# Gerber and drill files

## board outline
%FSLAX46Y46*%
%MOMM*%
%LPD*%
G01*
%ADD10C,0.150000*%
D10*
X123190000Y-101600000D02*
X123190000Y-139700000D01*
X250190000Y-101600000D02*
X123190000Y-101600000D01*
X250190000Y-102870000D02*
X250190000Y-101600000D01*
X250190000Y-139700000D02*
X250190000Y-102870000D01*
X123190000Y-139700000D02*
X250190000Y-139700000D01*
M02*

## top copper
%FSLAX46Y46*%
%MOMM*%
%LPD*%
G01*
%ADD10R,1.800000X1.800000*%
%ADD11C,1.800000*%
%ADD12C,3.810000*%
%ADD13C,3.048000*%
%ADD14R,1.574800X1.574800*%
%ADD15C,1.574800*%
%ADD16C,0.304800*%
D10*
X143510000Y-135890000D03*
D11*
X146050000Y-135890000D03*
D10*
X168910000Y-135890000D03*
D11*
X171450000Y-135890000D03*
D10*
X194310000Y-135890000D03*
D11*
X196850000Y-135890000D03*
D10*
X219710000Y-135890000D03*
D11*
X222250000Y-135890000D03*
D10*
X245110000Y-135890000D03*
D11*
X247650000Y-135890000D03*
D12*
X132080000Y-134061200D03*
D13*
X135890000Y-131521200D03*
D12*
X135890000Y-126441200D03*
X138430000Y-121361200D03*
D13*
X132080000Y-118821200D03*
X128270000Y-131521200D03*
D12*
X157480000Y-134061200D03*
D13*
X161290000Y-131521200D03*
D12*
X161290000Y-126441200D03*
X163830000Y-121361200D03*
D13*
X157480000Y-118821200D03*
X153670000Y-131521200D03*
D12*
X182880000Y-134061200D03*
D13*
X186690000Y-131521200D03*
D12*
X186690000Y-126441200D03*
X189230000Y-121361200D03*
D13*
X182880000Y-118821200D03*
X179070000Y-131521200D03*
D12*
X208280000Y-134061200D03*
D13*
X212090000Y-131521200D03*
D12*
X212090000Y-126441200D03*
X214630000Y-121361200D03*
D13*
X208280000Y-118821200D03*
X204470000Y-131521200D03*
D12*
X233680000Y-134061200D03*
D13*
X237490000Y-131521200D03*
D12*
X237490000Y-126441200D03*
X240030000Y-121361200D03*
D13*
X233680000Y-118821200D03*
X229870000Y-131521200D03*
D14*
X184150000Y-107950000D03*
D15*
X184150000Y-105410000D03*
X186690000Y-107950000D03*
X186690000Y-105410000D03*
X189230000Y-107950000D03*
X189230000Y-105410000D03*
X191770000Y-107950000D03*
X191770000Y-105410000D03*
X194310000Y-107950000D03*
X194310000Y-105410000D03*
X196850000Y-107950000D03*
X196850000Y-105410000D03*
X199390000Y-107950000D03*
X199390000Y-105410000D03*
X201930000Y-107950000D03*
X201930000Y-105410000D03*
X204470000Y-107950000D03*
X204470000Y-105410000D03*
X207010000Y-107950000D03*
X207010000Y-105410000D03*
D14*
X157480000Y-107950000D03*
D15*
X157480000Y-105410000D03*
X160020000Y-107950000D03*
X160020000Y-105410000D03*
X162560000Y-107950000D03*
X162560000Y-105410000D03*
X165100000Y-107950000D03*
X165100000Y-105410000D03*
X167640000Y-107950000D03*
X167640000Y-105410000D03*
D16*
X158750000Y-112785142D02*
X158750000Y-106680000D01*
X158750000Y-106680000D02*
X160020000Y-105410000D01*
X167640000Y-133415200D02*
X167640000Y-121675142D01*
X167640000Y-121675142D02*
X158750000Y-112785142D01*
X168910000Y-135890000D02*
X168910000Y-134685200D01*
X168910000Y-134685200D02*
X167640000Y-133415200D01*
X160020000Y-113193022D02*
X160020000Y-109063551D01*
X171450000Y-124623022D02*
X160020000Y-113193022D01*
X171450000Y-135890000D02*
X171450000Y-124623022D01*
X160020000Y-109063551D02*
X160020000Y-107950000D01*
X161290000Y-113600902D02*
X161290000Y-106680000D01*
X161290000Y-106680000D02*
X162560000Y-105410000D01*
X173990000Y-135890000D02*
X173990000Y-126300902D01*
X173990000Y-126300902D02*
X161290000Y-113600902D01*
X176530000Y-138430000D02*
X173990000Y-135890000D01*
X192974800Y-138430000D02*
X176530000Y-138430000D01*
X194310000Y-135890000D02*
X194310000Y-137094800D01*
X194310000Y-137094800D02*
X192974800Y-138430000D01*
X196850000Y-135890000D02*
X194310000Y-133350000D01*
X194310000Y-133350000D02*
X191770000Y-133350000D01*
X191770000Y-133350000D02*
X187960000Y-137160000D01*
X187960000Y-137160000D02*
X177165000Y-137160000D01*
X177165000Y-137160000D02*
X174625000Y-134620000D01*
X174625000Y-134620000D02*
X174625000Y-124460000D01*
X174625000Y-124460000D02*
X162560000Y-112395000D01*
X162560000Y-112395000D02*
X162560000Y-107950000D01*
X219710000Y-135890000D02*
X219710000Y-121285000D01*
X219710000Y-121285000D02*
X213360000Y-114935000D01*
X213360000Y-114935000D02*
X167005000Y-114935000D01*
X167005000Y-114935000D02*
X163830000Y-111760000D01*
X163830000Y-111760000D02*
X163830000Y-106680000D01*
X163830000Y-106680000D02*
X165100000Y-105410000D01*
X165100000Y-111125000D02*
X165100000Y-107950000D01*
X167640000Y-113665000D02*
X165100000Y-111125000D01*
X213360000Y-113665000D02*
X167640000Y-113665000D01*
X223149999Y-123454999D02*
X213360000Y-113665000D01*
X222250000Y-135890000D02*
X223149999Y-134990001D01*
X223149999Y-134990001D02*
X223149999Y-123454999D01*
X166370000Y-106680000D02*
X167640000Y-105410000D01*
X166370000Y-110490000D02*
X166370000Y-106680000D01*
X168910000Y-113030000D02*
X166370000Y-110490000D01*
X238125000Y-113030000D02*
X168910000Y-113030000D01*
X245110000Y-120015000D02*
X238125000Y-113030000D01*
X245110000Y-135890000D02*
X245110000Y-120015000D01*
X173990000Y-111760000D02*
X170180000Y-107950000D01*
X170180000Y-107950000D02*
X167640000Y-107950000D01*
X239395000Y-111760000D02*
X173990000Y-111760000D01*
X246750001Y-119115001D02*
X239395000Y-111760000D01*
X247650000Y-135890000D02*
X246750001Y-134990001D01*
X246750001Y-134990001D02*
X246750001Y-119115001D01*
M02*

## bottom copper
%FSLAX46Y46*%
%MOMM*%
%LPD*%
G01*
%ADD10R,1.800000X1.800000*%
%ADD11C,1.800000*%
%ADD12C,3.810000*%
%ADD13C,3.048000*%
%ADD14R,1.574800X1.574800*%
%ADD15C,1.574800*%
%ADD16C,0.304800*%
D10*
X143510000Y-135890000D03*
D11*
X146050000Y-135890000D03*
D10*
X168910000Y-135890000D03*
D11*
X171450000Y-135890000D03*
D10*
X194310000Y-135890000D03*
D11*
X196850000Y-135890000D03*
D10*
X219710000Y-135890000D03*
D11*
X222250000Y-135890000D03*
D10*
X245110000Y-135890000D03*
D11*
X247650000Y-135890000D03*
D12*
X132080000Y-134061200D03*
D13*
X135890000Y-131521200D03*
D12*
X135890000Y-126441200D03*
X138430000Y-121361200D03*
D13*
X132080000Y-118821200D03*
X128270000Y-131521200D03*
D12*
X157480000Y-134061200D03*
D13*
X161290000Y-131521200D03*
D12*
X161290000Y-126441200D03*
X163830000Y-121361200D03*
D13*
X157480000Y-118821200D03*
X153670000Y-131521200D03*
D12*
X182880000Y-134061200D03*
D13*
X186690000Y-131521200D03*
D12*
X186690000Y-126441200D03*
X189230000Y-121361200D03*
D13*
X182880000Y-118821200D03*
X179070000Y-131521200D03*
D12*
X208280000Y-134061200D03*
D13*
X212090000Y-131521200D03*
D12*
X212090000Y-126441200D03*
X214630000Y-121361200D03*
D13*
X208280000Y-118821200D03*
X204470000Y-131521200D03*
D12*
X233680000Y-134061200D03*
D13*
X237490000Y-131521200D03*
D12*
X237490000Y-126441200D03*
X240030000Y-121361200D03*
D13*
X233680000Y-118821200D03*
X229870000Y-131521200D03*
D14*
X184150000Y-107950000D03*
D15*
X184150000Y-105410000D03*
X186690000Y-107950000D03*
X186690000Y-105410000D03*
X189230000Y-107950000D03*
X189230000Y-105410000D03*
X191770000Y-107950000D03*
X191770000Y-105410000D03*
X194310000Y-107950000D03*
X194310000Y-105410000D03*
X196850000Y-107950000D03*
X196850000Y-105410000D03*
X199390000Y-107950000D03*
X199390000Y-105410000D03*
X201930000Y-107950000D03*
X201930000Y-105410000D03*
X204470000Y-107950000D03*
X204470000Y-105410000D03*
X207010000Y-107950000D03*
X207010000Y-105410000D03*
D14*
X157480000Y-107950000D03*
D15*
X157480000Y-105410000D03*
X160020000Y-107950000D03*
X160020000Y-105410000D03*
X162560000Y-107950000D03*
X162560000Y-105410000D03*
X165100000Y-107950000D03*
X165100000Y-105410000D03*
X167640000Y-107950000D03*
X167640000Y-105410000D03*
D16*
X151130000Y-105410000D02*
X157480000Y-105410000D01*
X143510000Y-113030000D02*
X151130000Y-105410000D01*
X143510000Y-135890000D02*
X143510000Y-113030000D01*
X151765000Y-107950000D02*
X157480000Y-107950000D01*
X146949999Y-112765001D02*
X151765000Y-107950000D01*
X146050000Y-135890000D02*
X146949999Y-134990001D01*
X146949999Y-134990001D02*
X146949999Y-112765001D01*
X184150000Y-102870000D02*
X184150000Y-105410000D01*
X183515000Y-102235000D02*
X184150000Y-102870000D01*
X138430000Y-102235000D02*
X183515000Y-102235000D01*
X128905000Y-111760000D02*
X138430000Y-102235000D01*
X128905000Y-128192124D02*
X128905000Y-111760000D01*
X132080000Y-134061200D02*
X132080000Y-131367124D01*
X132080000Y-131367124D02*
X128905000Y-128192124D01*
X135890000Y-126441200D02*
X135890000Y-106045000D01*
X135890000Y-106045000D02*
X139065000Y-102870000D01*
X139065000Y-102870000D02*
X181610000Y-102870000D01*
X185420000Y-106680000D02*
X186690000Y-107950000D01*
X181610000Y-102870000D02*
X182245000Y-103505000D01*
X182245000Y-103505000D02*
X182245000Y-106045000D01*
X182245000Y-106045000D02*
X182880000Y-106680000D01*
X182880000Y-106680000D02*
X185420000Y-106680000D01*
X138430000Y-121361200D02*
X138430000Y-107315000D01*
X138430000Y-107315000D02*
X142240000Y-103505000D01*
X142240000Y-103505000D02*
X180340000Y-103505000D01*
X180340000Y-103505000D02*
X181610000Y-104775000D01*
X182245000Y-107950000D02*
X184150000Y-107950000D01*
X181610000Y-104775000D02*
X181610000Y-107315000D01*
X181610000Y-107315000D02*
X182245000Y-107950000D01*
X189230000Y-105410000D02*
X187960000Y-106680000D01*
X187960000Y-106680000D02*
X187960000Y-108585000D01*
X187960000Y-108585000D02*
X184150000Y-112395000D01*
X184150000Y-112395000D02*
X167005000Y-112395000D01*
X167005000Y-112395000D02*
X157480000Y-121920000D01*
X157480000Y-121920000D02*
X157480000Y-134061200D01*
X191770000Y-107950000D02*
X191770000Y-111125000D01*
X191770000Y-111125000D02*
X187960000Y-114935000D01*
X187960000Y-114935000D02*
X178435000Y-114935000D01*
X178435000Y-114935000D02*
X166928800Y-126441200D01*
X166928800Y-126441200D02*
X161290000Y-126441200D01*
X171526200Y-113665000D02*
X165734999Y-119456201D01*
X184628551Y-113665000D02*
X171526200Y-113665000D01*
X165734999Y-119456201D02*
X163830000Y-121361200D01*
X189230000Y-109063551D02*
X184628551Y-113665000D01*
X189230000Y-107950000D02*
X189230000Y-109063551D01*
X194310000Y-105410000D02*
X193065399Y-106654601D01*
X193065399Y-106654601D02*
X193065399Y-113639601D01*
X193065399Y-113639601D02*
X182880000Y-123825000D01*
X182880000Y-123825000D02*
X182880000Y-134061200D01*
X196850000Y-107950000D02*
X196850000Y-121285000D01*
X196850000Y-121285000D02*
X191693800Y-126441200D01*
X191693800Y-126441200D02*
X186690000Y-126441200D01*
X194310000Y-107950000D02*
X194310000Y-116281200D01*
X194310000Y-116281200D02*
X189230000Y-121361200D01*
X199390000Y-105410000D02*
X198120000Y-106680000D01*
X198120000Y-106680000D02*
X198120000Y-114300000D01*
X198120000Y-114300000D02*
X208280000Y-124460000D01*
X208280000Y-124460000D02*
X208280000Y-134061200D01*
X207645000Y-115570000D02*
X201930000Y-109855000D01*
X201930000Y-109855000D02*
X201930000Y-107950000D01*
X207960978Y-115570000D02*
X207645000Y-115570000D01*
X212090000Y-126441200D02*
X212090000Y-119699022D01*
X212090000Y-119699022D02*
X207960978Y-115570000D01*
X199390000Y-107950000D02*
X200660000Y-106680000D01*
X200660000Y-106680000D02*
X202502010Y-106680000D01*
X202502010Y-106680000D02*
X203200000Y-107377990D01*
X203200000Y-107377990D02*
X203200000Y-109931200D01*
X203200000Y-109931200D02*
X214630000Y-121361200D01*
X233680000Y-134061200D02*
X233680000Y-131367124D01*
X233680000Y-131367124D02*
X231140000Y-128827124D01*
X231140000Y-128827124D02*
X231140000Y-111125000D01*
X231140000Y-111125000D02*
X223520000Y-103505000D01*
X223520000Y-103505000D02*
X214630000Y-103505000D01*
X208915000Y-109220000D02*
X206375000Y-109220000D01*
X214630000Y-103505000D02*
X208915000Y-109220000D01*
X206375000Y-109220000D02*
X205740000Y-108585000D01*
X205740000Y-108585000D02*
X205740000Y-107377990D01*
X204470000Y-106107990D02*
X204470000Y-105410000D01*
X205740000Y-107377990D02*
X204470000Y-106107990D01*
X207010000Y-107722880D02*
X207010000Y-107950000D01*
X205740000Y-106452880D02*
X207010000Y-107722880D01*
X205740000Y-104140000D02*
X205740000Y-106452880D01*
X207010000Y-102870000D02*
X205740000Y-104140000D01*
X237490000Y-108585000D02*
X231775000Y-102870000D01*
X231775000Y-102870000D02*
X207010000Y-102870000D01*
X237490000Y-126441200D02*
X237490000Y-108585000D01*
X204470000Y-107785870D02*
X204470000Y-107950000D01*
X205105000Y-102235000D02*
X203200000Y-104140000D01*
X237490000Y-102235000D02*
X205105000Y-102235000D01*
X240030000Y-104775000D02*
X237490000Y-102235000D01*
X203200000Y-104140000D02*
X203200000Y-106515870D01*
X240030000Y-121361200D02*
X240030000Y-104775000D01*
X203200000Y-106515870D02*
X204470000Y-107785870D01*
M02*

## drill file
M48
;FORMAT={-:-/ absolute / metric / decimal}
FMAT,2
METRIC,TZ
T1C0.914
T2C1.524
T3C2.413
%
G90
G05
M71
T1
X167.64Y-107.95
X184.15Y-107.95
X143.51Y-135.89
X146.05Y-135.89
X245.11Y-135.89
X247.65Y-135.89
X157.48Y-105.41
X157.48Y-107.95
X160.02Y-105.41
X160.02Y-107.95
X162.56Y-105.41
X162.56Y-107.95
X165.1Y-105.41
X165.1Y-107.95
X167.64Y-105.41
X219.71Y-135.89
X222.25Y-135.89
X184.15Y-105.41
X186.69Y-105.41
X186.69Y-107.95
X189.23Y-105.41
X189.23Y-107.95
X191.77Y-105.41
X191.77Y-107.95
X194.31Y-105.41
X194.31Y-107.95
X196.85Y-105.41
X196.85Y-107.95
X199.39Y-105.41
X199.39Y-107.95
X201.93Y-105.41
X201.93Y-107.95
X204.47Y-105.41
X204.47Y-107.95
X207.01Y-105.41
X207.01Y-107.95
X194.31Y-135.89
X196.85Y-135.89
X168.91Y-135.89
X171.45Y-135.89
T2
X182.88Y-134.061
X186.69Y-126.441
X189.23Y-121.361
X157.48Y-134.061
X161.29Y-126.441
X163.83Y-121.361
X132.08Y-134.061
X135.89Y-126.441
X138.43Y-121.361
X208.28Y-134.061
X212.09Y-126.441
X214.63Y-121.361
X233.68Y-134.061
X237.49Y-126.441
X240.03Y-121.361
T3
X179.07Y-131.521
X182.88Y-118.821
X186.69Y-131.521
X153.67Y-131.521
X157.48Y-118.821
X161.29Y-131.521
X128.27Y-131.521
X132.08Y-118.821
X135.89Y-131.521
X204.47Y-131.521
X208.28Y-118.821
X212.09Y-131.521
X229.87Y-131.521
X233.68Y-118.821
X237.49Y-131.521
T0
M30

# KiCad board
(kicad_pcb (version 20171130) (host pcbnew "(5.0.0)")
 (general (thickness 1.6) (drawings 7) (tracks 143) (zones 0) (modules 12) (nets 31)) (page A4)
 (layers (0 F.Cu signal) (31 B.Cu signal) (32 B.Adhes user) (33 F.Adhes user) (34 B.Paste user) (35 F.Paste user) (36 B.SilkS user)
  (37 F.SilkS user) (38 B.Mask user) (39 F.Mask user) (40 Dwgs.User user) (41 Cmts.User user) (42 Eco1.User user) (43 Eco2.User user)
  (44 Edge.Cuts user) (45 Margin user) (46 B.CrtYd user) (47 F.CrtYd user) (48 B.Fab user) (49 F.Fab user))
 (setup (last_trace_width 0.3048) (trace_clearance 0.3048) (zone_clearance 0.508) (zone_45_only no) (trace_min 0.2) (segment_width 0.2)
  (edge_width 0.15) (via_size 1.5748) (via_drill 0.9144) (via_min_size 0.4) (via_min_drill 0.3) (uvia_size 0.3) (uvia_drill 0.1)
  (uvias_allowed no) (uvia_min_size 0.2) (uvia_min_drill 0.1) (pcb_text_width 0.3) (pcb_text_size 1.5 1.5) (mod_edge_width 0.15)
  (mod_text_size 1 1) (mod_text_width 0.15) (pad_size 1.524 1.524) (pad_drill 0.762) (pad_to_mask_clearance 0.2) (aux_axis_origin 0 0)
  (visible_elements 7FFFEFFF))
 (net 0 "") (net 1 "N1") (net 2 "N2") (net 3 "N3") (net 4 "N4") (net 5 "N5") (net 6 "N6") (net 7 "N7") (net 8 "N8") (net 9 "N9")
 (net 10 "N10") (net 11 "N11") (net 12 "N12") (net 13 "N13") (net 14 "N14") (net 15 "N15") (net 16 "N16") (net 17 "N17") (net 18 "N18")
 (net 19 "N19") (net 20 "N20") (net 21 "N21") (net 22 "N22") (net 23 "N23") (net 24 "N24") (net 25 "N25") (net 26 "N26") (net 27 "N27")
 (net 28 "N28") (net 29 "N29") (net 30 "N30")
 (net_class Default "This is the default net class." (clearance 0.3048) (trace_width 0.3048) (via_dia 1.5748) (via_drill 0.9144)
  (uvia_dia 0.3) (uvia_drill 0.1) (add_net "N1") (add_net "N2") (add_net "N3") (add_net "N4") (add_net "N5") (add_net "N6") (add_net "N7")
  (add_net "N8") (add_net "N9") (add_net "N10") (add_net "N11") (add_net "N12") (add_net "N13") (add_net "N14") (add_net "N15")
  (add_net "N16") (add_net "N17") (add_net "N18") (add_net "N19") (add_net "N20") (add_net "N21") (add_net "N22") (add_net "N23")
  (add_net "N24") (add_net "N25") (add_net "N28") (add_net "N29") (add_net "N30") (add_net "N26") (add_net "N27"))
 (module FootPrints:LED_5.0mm (layer F.Cu) (at 143.51 135.89)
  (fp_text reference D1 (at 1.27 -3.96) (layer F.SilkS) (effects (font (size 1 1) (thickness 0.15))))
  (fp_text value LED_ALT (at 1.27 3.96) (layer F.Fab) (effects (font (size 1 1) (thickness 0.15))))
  (pad 1 thru_hole rect (at 0 0) (size 1.8 1.8) (drill 0.9144) (layers *.Cu *.Mask) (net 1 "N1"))
  (pad 2 thru_hole circle (at 2.54 0) (size 1.8 1.8) (drill 0.9144) (layers *.Cu *.Mask) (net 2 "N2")))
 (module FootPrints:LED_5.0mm (layer F.Cu) (at 168.91 135.89)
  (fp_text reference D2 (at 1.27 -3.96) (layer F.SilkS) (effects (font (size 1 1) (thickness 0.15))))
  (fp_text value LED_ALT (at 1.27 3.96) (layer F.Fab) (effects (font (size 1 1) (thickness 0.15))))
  (pad 1 thru_hole rect (at 0 0) (size 1.8 1.8) (drill 0.9144) (layers *.Cu *.Mask) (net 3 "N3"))
  (pad 2 thru_hole circle (at 2.54 0) (size 1.8 1.8) (drill 0.9144) (layers *.Cu *.Mask) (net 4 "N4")))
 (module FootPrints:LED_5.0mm (layer F.Cu) (at 194.31 135.89)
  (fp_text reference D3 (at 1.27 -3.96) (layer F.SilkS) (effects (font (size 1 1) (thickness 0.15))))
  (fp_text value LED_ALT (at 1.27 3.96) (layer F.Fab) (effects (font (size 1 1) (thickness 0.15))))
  (pad 1 thru_hole rect (at 0 0) (size 1.8 1.8) (drill 0.9144) (layers *.Cu *.Mask) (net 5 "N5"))
  (pad 2 thru_hole circle (at 2.54 0) (size 1.8 1.8) (drill 0.9144) (layers *.Cu *.Mask) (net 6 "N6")))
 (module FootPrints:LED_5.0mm (layer F.Cu) (at 219.71 135.89)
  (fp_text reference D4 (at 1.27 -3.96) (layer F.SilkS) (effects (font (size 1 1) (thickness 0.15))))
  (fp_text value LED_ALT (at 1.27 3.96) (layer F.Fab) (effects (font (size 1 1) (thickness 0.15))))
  (pad 1 thru_hole rect (at 0 0) (size 1.8 1.8) (drill 0.9144) (layers *.Cu *.Mask) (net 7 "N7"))
  (pad 2 thru_hole circle (at 2.54 0) (size 1.8 1.8) (drill 0.9144) (layers *.Cu *.Mask) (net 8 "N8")))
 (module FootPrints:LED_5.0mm (layer F.Cu) (at 245.11 135.89)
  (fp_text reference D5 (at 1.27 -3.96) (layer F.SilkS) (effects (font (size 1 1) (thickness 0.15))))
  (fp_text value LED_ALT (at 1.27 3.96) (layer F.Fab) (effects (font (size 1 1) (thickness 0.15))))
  (pad 1 thru_hole rect (at 0 0) (size 1.8 1.8) (drill 0.9144) (layers *.Cu *.Mask) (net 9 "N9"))
  (pad 2 thru_hole circle (at 2.54 0) (size 1.8 1.8) (drill 0.9144) (layers *.Cu *.Mask) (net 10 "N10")))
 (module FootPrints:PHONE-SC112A (layer F.Cu) (at 132.08 139.7 270)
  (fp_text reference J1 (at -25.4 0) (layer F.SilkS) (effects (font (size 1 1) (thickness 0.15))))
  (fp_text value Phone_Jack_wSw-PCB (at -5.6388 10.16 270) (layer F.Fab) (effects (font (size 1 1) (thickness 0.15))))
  (pad 1 thru_hole circle (at -5.6388 0 270) (size 3.81 3.81) (drill 1.524) (layers *.Cu *.Mask F.SilkS) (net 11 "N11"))
  (pad "" thru_hole circle (at -8.1788 -3.81 270) (size 3.048 3.048) (drill 2.413) (layers *.Cu *.Mask F.SilkS))
  (pad 2 thru_hole circle (at -13.2588 -3.81 270) (size 3.81 3.81) (drill 1.524) (layers *.Cu *.Mask F.SilkS) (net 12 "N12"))
  (pad 3 thru_hole circle (at -18.3388 -6.35 270) (size 3.81 3.81) (drill 1.524) (layers *.Cu *.Mask F.SilkS) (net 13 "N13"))
  (pad "" thru_hole circle (at -20.8788 0 270) (size 3.048 3.048) (drill 2.413) (layers *.Cu *.Mask F.SilkS))
  (pad "" thru_hole circle (at -8.1788 3.81 270) (size 3.048 3.048) (drill 2.413) (layers *.Cu *.Mask F.SilkS)))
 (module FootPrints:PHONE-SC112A (layer F.Cu) (at 157.48 139.7 270)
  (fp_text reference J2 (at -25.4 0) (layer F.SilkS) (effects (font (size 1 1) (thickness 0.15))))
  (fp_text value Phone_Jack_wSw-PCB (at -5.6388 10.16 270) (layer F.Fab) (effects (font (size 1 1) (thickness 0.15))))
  (pad 1 thru_hole circle (at -5.6388 0 270) (size 3.81 3.81) (drill 1.524) (layers *.Cu *.Mask F.SilkS) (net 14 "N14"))
  (pad "" thru_hole circle (at -8.1788 -3.81 270) (size 3.048 3.048) (drill 2.413) (layers *.Cu *.Mask F.SilkS))
  (pad 2 thru_hole circle (at -13.2588 -3.81 270) (size 3.81 3.81) (drill 1.524) (layers *.Cu *.Mask F.SilkS) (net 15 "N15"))
  (pad 3 thru_hole circle (at -18.3388 -6.35 270) (size 3.81 3.81) (drill 1.524) (layers *.Cu *.Mask F.SilkS) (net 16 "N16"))
  (pad "" thru_hole circle (at -20.8788 0 270) (size 3.048 3.048) (drill 2.413) (layers *.Cu *.Mask F.SilkS))
  (pad "" thru_hole circle (at -8.1788 3.81 270) (size 3.048 3.048) (drill 2.413) (layers *.Cu *.Mask F.SilkS)))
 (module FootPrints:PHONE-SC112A (layer F.Cu) (at 182.88 139.7 270)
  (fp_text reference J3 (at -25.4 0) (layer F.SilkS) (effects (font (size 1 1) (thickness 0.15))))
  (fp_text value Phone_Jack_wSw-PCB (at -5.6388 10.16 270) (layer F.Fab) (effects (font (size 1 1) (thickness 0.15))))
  (pad 1 thru_hole circle (at -5.6388 0 270) (size 3.81 3.81) (drill 1.524) (layers *.Cu *.Mask F.SilkS) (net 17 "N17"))
  (pad "" thru_hole circle (at -8.1788 -3.81 270) (size 3.048 3.048) (drill 2.413) (layers *.Cu *.Mask F.SilkS))
  (pad 2 thru_hole circle (at -13.2588 -3.81 270) (size 3.81 3.81) (drill 1.524) (layers *.Cu *.Mask F.SilkS) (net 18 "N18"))
  (pad 3 thru_hole circle (at -18.3388 -6.35 270) (size 3.81 3.81) (drill 1.524) (layers *.Cu *.Mask F.SilkS) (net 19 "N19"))
  (pad "" thru_hole circle (at -20.8788 0 270) (size 3.048 3.048) (drill 2.413) (layers *.Cu *.Mask F.SilkS))
  (pad "" thru_hole circle (at -8.1788 3.81 270) (size 3.048 3.048) (drill 2.413) (layers *.Cu *.Mask F.SilkS)))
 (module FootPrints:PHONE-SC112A (layer F.Cu) (at 208.28 139.7 270)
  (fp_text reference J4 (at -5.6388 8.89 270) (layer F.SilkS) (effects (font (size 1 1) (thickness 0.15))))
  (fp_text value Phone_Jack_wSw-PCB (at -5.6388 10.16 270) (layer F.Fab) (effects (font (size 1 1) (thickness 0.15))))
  (pad 1 thru_hole circle (at -5.6388 0 270) (size 3.81 3.81) (drill 1.524) (layers *.Cu *.Mask F.SilkS) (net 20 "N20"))
  (pad "" thru_hole circle (at -8.1788 -3.81 270) (size 3.048 3.048) (drill 2.413) (layers *.Cu *.Mask F.SilkS))
  (pad 2 thru_hole circle (at -13.2588 -3.81 270) (size 3.81 3.81) (drill 1.524) (layers *.Cu *.Mask F.SilkS) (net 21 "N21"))
  (pad 3 thru_hole circle (at -18.3388 -6.35 270) (size 3.81 3.81) (drill 1.524) (layers *.Cu *.Mask F.SilkS) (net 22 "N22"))
  (pad "" thru_hole circle (at -20.8788 0 270) (size 3.048 3.048) (drill 2.413) (layers *.Cu *.Mask F.SilkS))
  (pad "" thru_hole circle (at -8.1788 3.81 270) (size 3.048 3.048) (drill 2.413) (layers *.Cu *.Mask F.SilkS)))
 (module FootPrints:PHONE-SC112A (layer F.Cu) (at 233.68 139.7 270)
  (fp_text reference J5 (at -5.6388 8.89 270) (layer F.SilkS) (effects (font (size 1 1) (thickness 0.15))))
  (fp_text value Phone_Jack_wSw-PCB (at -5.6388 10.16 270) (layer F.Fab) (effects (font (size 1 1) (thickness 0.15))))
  (pad 1 thru_hole circle (at -5.6388 0 270) (size 3.81 3.81) (drill 1.524) (layers *.Cu *.Mask F.SilkS) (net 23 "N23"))
  (pad "" thru_hole circle (at -8.1788 -3.81 270) (size 3.048 3.048) (drill 2.413) (layers *.Cu *.Mask F.SilkS))
  (pad 2 thru_hole circle (at -13.2588 -3.81 270) (size 3.81 3.81) (drill 1.524) (layers *.Cu *.Mask F.SilkS) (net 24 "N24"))
  (pad 3 thru_hole circle (at -18.3388 -6.35 270) (size 3.81 3.81) (drill 1.524) (layers *.Cu *.Mask F.SilkS) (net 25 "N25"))
  (pad "" thru_hole circle (at -20.8788 0 270) (size 3.048 3.048) (drill 2.413) (layers *.Cu *.Mask F.SilkS))
  (pad "" thru_hole circle (at -8.1788 3.81 270) (size 3.048 3.048) (drill 2.413) (layers *.Cu *.Mask F.SilkS)))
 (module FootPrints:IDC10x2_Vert (layer F.Cu) (at 195.58 106.68)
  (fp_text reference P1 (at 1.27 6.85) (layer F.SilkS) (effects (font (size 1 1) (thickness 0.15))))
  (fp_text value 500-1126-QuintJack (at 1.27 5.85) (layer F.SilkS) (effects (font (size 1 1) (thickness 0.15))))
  (pad 1 thru_hole rect (at -11.43 1.27) (size 1.5748 1.5748) (drill 0.9144) (layers *.Cu *.Mask) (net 13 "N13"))
  (pad 2 thru_hole circle (at -11.43 -1.27) (size 1.5748 1.5748) (drill 0.9144) (layers *.Cu *.Mask) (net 11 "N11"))
  (pad 3 thru_hole circle (at -8.89 1.27) (size 1.5748 1.5748) (drill 0.9144) (layers *.Cu *.Mask) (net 12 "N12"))
  (pad 4 thru_hole circle (at -8.89 -1.27) (size 1.5748 1.5748) (drill 0.9144) (layers *.Cu *.Mask) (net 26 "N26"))
  (pad 5 thru_hole circle (at -6.35 1.27) (size 1.5748 1.5748) (drill 0.9144) (layers *.Cu *.Mask) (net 16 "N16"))
  (pad 6 thru_hole circle (at -6.35 -1.27) (size 1.5748 1.5748) (drill 0.9144) (layers *.Cu *.Mask) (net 14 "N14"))
  (pad 7 thru_hole circle (at -3.81 1.27) (size 1.5748 1.5748) (drill 0.9144) (layers *.Cu *.Mask) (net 15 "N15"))
  (pad 8 thru_hole circle (at -3.81 -1.27) (size 1.5748 1.5748) (drill 0.9144) (layers *.Cu *.Mask) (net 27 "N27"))
  (pad 9 thru_hole circle (at -1.27 1.27) (size 1.5748 1.5748) (drill 0.9144) (layers *.Cu *.Mask) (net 19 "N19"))
  (pad 10 thru_hole circle (at -1.27 -1.27) (size 1.5748 1.5748) (drill 0.9144) (layers *.Cu *.Mask) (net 17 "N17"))
  (pad 11 thru_hole circle (at 1.27 1.27) (size 1.5748 1.5748) (drill 0.9144) (layers *.Cu *.Mask) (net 18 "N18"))
  (pad 12 thru_hole circle (at 1.27 -1.27) (size 1.5748 1.5748) (drill 0.9144) (layers *.Cu *.Mask) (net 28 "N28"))
  (pad 13 thru_hole circle (at 3.81 1.27) (size 1.5748 1.5748) (drill 0.9144) (layers *.Cu *.Mask) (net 22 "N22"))
  (pad 14 thru_hole circle (at 3.81 -1.27) (size 1.5748 1.5748) (drill 0.9144) (layers *.Cu *.Mask) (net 20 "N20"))
  (pad 15 thru_hole circle (at 6.35 1.27) (size 1.5748 1.5748) (drill 0.9144) (layers *.Cu *.Mask) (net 21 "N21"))
  (pad 16 thru_hole circle (at 6.35 -1.27) (size 1.5748 1.5748) (drill 0.9144) (layers *.Cu *.Mask) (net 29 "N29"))
  (pad 17 thru_hole circle (at 8.89 1.27) (size 1.5748 1.5748) (drill 0.9144) (layers *.Cu *.Mask) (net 25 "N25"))
  (pad 18 thru_hole circle (at 8.89 -1.27) (size 1.5748 1.5748) (drill 0.9144) (layers *.Cu *.Mask) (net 23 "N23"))
  (pad 19 thru_hole circle (at 11.43 1.27) (size 1.5748 1.5748) (drill 0.9144) (layers *.Cu *.Mask) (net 24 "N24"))
  (pad 20 thru_hole circle (at 11.43 -1.27) (size 1.5748 1.5748) (drill 0.9144) (layers *.Cu *.Mask) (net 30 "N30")))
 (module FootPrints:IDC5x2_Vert (layer F.Cu) (at 162.56 106.68 180)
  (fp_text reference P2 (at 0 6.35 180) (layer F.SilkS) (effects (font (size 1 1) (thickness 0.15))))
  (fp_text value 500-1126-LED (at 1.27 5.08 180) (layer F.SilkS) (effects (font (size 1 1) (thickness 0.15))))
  (pad 1 thru_hole rect (at 5.08 -1.27 180) (size 1.5748 1.5748) (drill 0.9144) (layers *.Cu *.Mask F.SilkS) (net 2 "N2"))
  (pad 2 thru_hole circle (at 5.08 1.27 180) (size 1.5748 1.5748) (drill 0.9144) (layers *.Cu *.Mask F.SilkS) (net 1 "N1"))
  (pad 3 thru_hole circle (at 2.54 -1.27 180) (size 1.5748 1.5748) (drill 0.9144) (layers *.Cu *.Mask F.SilkS) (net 4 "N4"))
  (pad 4 thru_hole circle (at 2.54 1.27 180) (size 1.5748 1.5748) (drill 0.9144) (layers *.Cu *.Mask F.SilkS) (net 3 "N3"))
  (pad 5 thru_hole circle (at 0 -1.27 180) (size 1.5748 1.5748) (drill 0.9144) (layers *.Cu *.Mask F.SilkS) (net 6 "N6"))
  (pad 6 thru_hole circle (at 0 1.27 180) (size 1.5748 1.5748) (drill 0.9144) (layers *.Cu *.Mask F.SilkS) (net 5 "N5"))
  (pad 7 thru_hole circle (at -2.54 -1.27 180) (size 1.5748 1.5748) (drill 0.9144) (layers *.Cu *.Mask F.SilkS) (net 8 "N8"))
  (pad 8 thru_hole circle (at -2.54 1.27 180) (size 1.5748 1.5748) (drill 0.9144) (layers *.Cu *.Mask F.SilkS) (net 7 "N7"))
  (pad 9 thru_hole circle (at -5.08 -1.27 180) (size 1.5748 1.5748) (drill 0.9144) (layers *.Cu *.Mask F.SilkS) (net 10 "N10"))
  (pad 10 thru_hole circle (at -5.08 1.27 180) (size 1.5748 1.5748) (drill 0.9144) (layers *.Cu *.Mask F.SilkS) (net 9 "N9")))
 (gr_line (start 123.19 101.6) (end 123.19 139.7) (angle 90) (layer Edge.Cuts) (width 0.15))
 (gr_line (start 250.19 101.6) (end 123.19 101.6) (angle 90) (layer Edge.Cuts) (width 0.15))
 (gr_line (start 250.19 102.87) (end 250.19 101.6) (angle 90) (layer Edge.Cuts) (width 0.15))
 (gr_line (start 250.19 139.7) (end 250.19 102.87) (angle 90) (layer Edge.Cuts) (width 0.15))
 (gr_line (start 123.19 139.7) (end 250.19 139.7) (angle 90) (layer Edge.Cuts) (width 0.15))
 (segment (start 151.13 105.41) (end 157.48 105.41) (width 0.3048) (layer B.Cu) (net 1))
 (segment (start 143.51 113.03) (end 151.13 105.41) (width 0.3048) (layer B.Cu) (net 1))
 (segment (start 143.51 135.89) (end 143.51 113.03) (width 0.3048) (layer B.Cu) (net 1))
 (segment (start 151.765 107.95) (end 157.48 107.95) (width 0.3048) (layer B.Cu) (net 2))
 (segment (start 146.949999 112.765001) (end 151.765 107.95) (width 0.3048) (layer B.Cu) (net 2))
 (segment (start 146.05 135.89) (end 146.949999 134.990001) (width 0.3048) (layer B.Cu) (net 2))
 (segment (start 146.949999 134.990001) (end 146.949999 112.765001) (width 0.3048) (layer B.Cu) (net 2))
 (segment (start 158.75 112.785142) (end 158.75 106.68) (width 0.3048) (layer F.Cu) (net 3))
 (segment (start 158.75 106.68) (end 160.02 105.41) (width 0.3048) (layer F.Cu) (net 3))
 (segment (start 167.64 133.4152) (end 167.64 121.675142) (width 0.3048) (layer F.Cu) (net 3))
 (segment (start 167.64 121.675142) (end 158.75 112.785142) (width 0.3048) (layer F.Cu) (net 3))
 (segment (start 168.91 135.89) (end 168.91 134.6852) (width 0.3048) (layer F.Cu) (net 3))
 (segment (start 168.91 134.6852) (end 167.64 133.4152) (width 0.3048) (layer F.Cu) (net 3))
 (segment (start 160.02 113.193022) (end 160.02 109.063551) (width 0.3048) (layer F.Cu) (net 4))
 (segment (start 171.45 124.623022) (end 160.02 113.193022) (width 0.3048) (layer F.Cu) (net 4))
 (segment (start 171.45 135.89) (end 171.45 124.623022) (width 0.3048) (layer F.Cu) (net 4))
 (segment (start 160.02 109.063551) (end 160.02 107.95) (width 0.3048) (layer F.Cu) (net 4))
 (segment (start 161.29 113.600902) (end 161.29 106.68) (width 0.3048) (layer F.Cu) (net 5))
 (segment (start 161.29 106.68) (end 162.56 105.41) (width 0.3048) (layer F.Cu) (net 5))
 (segment (start 173.99 135.89) (end 173.99 126.300902) (width 0.3048) (layer F.Cu) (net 5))
 (segment (start 173.99 126.300902) (end 161.29 113.600902) (width 0.3048) (layer F.Cu) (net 5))
 (segment (start 176.53 138.43) (end 173.99 135.89) (width 0.3048) (layer F.Cu) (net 5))
 (segment (start 192.9748 138.43) (end 176.53 138.43) (width 0.3048) (layer F.Cu) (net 5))
 (segment (start 194.31 135.89) (end 194.31 137.0948) (width 0.3048) (layer F.Cu) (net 5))
 (segment (start 194.31 137.0948) (end 192.9748 138.43) (width 0.3048) (layer F.Cu) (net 5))
 (segment (start 196.85 135.89) (end 194.31 133.35) (width 0.3048) (layer F.Cu) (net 6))
 (segment (start 194.31 133.35) (end 191.77 133.35) (width 0.3048) (layer F.Cu) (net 6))
 (segment (start 191.77 133.35) (end 187.96 137.16) (width 0.3048) (layer F.Cu) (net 6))
 (segment (start 187.96 137.16) (end 177.165 137.16) (width 0.3048) (layer F.Cu) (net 6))
 (segment (start 177.165 137.16) (end 174.625 134.62) (width 0.3048) (layer F.Cu) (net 6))
 (segment (start 174.625 134.62) (end 174.625 124.46) (width 0.3048) (layer F.Cu) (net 6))
 (segment (start 174.625 124.46) (end 162.56 112.395) (width 0.3048) (layer F.Cu) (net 6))
 (segment (start 162.56 112.395) (end 162.56 107.95) (width 0.3048) (layer F.Cu) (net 6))
 (segment (start 219.71 135.89) (end 219.71 121.285) (width 0.3048) (layer F.Cu) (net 7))
 (segment (start 219.71 121.285) (end 213.36 114.935) (width 0.3048) (layer F.Cu) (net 7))
 (segment (start 213.36 114.935) (end 167.005 114.935) (width 0.3048) (layer F.Cu) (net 7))
 (segment (start 167.005 114.935) (end 163.83 111.76) (width 0.3048) (layer F.Cu) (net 7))
 (segment (start 163.83 111.76) (end 163.83 106.68) (width 0.3048) (layer F.Cu) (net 7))
 (segment (start 163.83 106.68) (end 165.1 105.41) (width 0.3048) (layer F.Cu) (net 7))
 (segment (start 165.1 111.125) (end 165.1 107.95) (width 0.3048) (layer F.Cu) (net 8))
 (segment (start 167.64 113.665) (end 165.1 111.125) (width 0.3048) (layer F.Cu) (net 8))
 (segment (start 213.36 113.665) (end 167.64 113.665) (width 0.3048) (layer F.Cu) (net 8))
 (segment (start 223.149999 123.454999) (end 213.36 113.665) (width 0.3048) (layer F.Cu) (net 8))
 (segment (start 222.25 135.89) (end 223.149999 134.990001) (width 0.3048) (layer F.Cu) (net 8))
 (segment (start 223.149999 134.990001) (end 223.149999 123.454999) (width 0.3048) (layer F.Cu) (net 8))
 (segment (start 166.37 106.68) (end 167.64 105.41) (width 0.3048) (layer F.Cu) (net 9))
 (segment (start 166.37 110.49) (end 166.37 106.68) (width 0.3048) (layer F.Cu) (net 9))
 (segment (start 168.91 113.03) (end 166.37 110.49) (width 0.3048) (layer F.Cu) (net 9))
 (segment (start 238.125 113.03) (end 168.91 113.03) (width 0.3048) (layer F.Cu) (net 9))
 (segment (start 245.11 120.015) (end 238.125 113.03) (width 0.3048) (layer F.Cu) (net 9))
 (segment (start 245.11 135.89) (end 245.11 120.015) (width 0.3048) (layer F.Cu) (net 9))
 (segment (start 173.99 111.76) (end 170.18 107.95) (width 0.3048) (layer F.Cu) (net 10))
 (segment (start 170.18 107.95) (end 167.64 107.95) (width 0.3048) (layer F.Cu) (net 10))
 (segment (start 239.395 111.76) (end 173.99 111.76) (width 0.3048) (layer F.Cu) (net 10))
 (segment (start 246.750001 119.115001) (end 239.395 111.76) (width 0.3048) (layer F.Cu) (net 10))
 (segment (start 247.65 135.89) (end 246.750001 134.990001) (width 0.3048) (layer F.Cu) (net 10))
 (segment (start 246.750001 134.990001) (end 246.750001 119.115001) (width 0.3048) (layer F.Cu) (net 10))
 (segment (start 184.15 102.87) (end 184.15 105.41) (width 0.3048) (layer B.Cu) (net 11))
 (segment (start 183.515 102.235) (end 184.15 102.87) (width 0.3048) (layer B.Cu) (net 11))
 (segment (start 138.43 102.235) (end 183.515 102.235) (width 0.3048) (layer B.Cu) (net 11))
 (segment (start 128.905 111.76) (end 138.43 102.235) (width 0.3048) (layer B.Cu) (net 11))
 (segment (start 128.905 128.192124) (end 128.905 111.76) (width 0.3048) (layer B.Cu) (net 11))
 (segment (start 132.08 134.0612) (end 132.08 131.367124) (width 0.3048) (layer B.Cu) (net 11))
 (segment (start 132.08 131.367124) (end 128.905 128.192124) (width 0.3048) (layer B.Cu) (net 11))
 (segment (start 135.89 126.4412) (end 135.89 106.045) (width 0.3048) (layer B.Cu) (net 12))
 (segment (start 135.89 106.045) (end 139.065 102.87) (width 0.3048) (layer B.Cu) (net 12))
 (segment (start 139.065 102.87) (end 181.61 102.87) (width 0.3048) (layer B.Cu) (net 12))
 (segment (start 185.42 106.68) (end 186.69 107.95) (width 0.3048) (layer B.Cu) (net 12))
 (segment (start 181.61 102.87) (end 182.245 103.505) (width 0.3048) (layer B.Cu) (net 12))
 (segment (start 182.245 103.505) (end 182.245 106.045) (width 0.3048) (layer B.Cu) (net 12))
 (segment (start 182.245 106.045) (end 182.88 106.68) (width 0.3048) (layer B.Cu) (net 12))
 (segment (start 182.88 106.68) (end 185.42 106.68) (width 0.3048) (layer B.Cu) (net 12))
 (segment (start 138.43 121.3612) (end 138.43 107.315) (width 0.3048) (layer B.Cu) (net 13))
 (segment (start 138.43 107.315) (end 142.24 103.505) (width 0.3048) (layer B.Cu) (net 13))
 (segment (start 142.24 103.505) (end 180.34 103.505) (width 0.3048) (layer B.Cu) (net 13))
 (segment (start 180.34 103.505) (end 181.61 104.775) (width 0.3048) (layer B.Cu) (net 13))
 (segment (start 182.245 107.95) (end 184.15 107.95) (width 0.3048) (layer B.Cu) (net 13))
 (segment (start 181.61 104.775) (end 181.61 107.315) (width 0.3048) (layer B.Cu) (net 13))
 (segment (start 181.61 107.315) (end 182.245 107.95) (width 0.3048) (layer B.Cu) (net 13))
 (segment (start 189.23 105.41) (end 187.96 106.68) (width 0.3048) (layer B.Cu) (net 14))
 (segment (start 187.96 106.68) (end 187.96 108.585) (width 0.3048) (layer B.Cu) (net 14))
 (segment (start 187.96 108.585) (end 184.15 112.395) (width 0.3048) (layer B.Cu) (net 14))
 (segment (start 184.15 112.395) (end 167.005 112.395) (width 0.3048) (layer B.Cu) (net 14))
 (segment (start 167.005 112.395) (end 157.48 121.92) (width 0.3048) (layer B.Cu) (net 14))
 (segment (start 157.48 121.92) (end 157.48 134.0612) (width 0.3048) (layer B.Cu) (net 14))
 (segment (start 191.77 107.95) (end 191.77 111.125) (width 0.3048) (layer B.Cu) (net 15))
 (segment (start 191.77 111.125) (end 187.96 114.935) (width 0.3048) (layer B.Cu) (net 15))
 (segment (start 187.96 114.935) (end 178.435 114.935) (width 0.3048) (layer B.Cu) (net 15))
 (segment (start 178.435 114.935) (end 166.9288 126.4412) (width 0.3048) (layer B.Cu) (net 15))
 (segment (start 166.9288 126.4412) (end 161.29 126.4412) (width 0.3048) (layer B.Cu) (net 15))
 (segment (start 171.5262 113.665) (end 165.734999 119.456201) (width 0.3048) (layer B.Cu) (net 16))
 (segment (start 184.628551 113.665) (end 171.5262 113.665) (width 0.3048) (layer B.Cu) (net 16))
 (segment (start 165.734999 119.456201) (end 163.83 121.3612) (width 0.3048) (layer B.Cu) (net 16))
 (segment (start 189.23 109.063551) (end 184.628551 113.665) (width 0.3048) (layer B.Cu) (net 16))
 (segment (start 189.23 107.95) (end 189.23 109.063551) (width 0.3048) (layer B.Cu) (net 16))
 (segment (start 194.31 105.41) (end 193.065399 106.654601) (width 0.3048) (layer B.Cu) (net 17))
 (segment (start 193.065399 106.654601) (end 193.065399 113.639601) (width 0.3048) (layer B.Cu) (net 17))
 (segment (start 193.065399 113.639601) (end 182.88 123.825) (width 0.3048) (layer B.Cu) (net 17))
 (segment (start 182.88 123.825) (end 182.88 134.0612) (width 0.3048) (layer B.Cu) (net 17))
 (segment (start 196.85 107.95) (end 196.85 121.285) (width 0.3048) (layer B.Cu) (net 18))
 (segment (start 196.85 121.285) (end 191.6938 126.4412) (width 0.3048) (layer B.Cu) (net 18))
 (segment (start 191.6938 126.4412) (end 186.69 126.4412) (width 0.3048) (layer B.Cu) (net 18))
 (segment (start 194.31 107.95) (end 194.31 116.2812) (width 0.3048) (layer B.Cu) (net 19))
 (segment (start 194.31 116.2812) (end 189.23 121.3612) (width 0.3048) (layer B.Cu) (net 19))
 (segment (start 199.39 105.41) (end 198.12 106.68) (width 0.3048) (layer B.Cu) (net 20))
 (segment (start 198.12 106.68) (end 198.12 114.3) (width 0.3048) (layer B.Cu) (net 20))
 (segment (start 198.12 114.3) (end 208.28 124.46) (width 0.3048) (layer B.Cu) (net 20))
 (segment (start 208.28 124.46) (end 208.28 134.0612) (width 0.3048) (layer B.Cu) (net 20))
 (segment (start 207.645 115.57) (end 201.93 109.855) (width 0.3048) (layer B.Cu) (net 21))
 (segment (start 201.93 109.855) (end 201.93 107.95) (width 0.3048) (layer B.Cu) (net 21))
 (segment (start 207.960978 115.57) (end 207.645 115.57) (width 0.3048) (layer B.Cu) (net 21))
 (segment (start 212.09 126.4412) (end 212.09 119.699022) (width 0.3048) (layer B.Cu) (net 21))
 (segment (start 212.09 119.699022) (end 207.960978 115.57) (width 0.3048) (layer B.Cu) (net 21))
 (segment (start 199.39 107.95) (end 200.66 106.68) (width 0.3048) (layer B.Cu) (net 22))
 (segment (start 200.66 106.68) (end 202.50201 106.68) (width 0.3048) (layer B.Cu) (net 22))
 (segment (start 202.50201 106.68) (end 203.2 107.37799) (width 0.3048) (layer B.Cu) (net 22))
 (segment (start 203.2 107.37799) (end 203.2 109.9312) (width 0.3048) (layer B.Cu) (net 22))
 (segment (start 203.2 109.9312) (end 214.63 121.3612) (width 0.3048) (layer B.Cu) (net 22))
 (segment (start 233.68 134.0612) (end 233.68 131.367124) (width 0.3048) (layer B.Cu) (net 23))
 (segment (start 233.68 131.367124) (end 231.14 128.827124) (width 0.3048) (layer B.Cu) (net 23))
 (segment (start 231.14 128.827124) (end 231.14 111.125) (width 0.3048) (layer B.Cu) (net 23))
 (segment (start 231.14 111.125) (end 223.52 103.505) (width 0.3048) (layer B.Cu) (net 23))
 (segment (start 223.52 103.505) (end 214.63 103.505) (width 0.3048) (layer B.Cu) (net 23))
 (segment (start 208.915 109.22) (end 206.375 109.22) (width 0.3048) (layer B.Cu) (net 23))
 (segment (start 214.63 103.505) (end 208.915 109.22) (width 0.3048) (layer B.Cu) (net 23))
 (segment (start 206.375 109.22) (end 205.74 108.585) (width 0.3048) (layer B.Cu) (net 23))
 (segment (start 205.74 108.585) (end 205.74 107.37799) (width 0.3048) (layer B.Cu) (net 23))
 (segment (start 204.47 106.10799) (end 204.47 105.41) (width 0.3048) (layer B.Cu) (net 23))
 (segment (start 205.74 107.37799) (end 204.47 106.10799) (width 0.3048) (layer B.Cu) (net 23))
 (segment (start 207.01 107.72288) (end 207.01 107.95) (width 0.3048) (layer B.Cu) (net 24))
 (segment (start 205.74 106.45288) (end 207.01 107.72288) (width 0.3048) (layer B.Cu) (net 24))
 (segment (start 205.74 104.14) (end 205.74 106.45288) (width 0.3048) (layer B.Cu) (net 24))
 (segment (start 207.01 102.87) (end 205.74 104.14) (width 0.3048) (layer B.Cu) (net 24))
 (segment (start 237.49 108.585) (end 231.775 102.87) (width 0.3048) (layer B.Cu) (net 24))
 (segment (start 231.775 102.87) (end 207.01 102.87) (width 0.3048) (layer B.Cu) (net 24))
 (segment (start 237.49 126.4412) (end 237.49 108.585) (width 0.3048) (layer B.Cu) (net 24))
 (segment (start 204.47 107.78587) (end 204.47 107.95) (width 0.3048) (layer B.Cu) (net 25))
 (segment (start 205.105 102.235) (end 203.2 104.14) (width 0.3048) (layer B.Cu) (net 25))
 (segment (start 237.49 102.235) (end 205.105 102.235) (width 0.3048) (layer B.Cu) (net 25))
 (segment (start 240.03 104.775) (end 237.49 102.235) (width 0.3048) (layer B.Cu) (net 25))
 (segment (start 203.2 104.14) (end 203.2 106.51587) (width 0.3048) (layer B.Cu) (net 25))
 (segment (start 240.03 121.3612) (end 240.03 104.775) (width 0.3048) (layer B.Cu) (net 25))
 (segment (start 203.2 106.51587) (end 204.47 107.78587) (width 0.3048) (layer B.Cu) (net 25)))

